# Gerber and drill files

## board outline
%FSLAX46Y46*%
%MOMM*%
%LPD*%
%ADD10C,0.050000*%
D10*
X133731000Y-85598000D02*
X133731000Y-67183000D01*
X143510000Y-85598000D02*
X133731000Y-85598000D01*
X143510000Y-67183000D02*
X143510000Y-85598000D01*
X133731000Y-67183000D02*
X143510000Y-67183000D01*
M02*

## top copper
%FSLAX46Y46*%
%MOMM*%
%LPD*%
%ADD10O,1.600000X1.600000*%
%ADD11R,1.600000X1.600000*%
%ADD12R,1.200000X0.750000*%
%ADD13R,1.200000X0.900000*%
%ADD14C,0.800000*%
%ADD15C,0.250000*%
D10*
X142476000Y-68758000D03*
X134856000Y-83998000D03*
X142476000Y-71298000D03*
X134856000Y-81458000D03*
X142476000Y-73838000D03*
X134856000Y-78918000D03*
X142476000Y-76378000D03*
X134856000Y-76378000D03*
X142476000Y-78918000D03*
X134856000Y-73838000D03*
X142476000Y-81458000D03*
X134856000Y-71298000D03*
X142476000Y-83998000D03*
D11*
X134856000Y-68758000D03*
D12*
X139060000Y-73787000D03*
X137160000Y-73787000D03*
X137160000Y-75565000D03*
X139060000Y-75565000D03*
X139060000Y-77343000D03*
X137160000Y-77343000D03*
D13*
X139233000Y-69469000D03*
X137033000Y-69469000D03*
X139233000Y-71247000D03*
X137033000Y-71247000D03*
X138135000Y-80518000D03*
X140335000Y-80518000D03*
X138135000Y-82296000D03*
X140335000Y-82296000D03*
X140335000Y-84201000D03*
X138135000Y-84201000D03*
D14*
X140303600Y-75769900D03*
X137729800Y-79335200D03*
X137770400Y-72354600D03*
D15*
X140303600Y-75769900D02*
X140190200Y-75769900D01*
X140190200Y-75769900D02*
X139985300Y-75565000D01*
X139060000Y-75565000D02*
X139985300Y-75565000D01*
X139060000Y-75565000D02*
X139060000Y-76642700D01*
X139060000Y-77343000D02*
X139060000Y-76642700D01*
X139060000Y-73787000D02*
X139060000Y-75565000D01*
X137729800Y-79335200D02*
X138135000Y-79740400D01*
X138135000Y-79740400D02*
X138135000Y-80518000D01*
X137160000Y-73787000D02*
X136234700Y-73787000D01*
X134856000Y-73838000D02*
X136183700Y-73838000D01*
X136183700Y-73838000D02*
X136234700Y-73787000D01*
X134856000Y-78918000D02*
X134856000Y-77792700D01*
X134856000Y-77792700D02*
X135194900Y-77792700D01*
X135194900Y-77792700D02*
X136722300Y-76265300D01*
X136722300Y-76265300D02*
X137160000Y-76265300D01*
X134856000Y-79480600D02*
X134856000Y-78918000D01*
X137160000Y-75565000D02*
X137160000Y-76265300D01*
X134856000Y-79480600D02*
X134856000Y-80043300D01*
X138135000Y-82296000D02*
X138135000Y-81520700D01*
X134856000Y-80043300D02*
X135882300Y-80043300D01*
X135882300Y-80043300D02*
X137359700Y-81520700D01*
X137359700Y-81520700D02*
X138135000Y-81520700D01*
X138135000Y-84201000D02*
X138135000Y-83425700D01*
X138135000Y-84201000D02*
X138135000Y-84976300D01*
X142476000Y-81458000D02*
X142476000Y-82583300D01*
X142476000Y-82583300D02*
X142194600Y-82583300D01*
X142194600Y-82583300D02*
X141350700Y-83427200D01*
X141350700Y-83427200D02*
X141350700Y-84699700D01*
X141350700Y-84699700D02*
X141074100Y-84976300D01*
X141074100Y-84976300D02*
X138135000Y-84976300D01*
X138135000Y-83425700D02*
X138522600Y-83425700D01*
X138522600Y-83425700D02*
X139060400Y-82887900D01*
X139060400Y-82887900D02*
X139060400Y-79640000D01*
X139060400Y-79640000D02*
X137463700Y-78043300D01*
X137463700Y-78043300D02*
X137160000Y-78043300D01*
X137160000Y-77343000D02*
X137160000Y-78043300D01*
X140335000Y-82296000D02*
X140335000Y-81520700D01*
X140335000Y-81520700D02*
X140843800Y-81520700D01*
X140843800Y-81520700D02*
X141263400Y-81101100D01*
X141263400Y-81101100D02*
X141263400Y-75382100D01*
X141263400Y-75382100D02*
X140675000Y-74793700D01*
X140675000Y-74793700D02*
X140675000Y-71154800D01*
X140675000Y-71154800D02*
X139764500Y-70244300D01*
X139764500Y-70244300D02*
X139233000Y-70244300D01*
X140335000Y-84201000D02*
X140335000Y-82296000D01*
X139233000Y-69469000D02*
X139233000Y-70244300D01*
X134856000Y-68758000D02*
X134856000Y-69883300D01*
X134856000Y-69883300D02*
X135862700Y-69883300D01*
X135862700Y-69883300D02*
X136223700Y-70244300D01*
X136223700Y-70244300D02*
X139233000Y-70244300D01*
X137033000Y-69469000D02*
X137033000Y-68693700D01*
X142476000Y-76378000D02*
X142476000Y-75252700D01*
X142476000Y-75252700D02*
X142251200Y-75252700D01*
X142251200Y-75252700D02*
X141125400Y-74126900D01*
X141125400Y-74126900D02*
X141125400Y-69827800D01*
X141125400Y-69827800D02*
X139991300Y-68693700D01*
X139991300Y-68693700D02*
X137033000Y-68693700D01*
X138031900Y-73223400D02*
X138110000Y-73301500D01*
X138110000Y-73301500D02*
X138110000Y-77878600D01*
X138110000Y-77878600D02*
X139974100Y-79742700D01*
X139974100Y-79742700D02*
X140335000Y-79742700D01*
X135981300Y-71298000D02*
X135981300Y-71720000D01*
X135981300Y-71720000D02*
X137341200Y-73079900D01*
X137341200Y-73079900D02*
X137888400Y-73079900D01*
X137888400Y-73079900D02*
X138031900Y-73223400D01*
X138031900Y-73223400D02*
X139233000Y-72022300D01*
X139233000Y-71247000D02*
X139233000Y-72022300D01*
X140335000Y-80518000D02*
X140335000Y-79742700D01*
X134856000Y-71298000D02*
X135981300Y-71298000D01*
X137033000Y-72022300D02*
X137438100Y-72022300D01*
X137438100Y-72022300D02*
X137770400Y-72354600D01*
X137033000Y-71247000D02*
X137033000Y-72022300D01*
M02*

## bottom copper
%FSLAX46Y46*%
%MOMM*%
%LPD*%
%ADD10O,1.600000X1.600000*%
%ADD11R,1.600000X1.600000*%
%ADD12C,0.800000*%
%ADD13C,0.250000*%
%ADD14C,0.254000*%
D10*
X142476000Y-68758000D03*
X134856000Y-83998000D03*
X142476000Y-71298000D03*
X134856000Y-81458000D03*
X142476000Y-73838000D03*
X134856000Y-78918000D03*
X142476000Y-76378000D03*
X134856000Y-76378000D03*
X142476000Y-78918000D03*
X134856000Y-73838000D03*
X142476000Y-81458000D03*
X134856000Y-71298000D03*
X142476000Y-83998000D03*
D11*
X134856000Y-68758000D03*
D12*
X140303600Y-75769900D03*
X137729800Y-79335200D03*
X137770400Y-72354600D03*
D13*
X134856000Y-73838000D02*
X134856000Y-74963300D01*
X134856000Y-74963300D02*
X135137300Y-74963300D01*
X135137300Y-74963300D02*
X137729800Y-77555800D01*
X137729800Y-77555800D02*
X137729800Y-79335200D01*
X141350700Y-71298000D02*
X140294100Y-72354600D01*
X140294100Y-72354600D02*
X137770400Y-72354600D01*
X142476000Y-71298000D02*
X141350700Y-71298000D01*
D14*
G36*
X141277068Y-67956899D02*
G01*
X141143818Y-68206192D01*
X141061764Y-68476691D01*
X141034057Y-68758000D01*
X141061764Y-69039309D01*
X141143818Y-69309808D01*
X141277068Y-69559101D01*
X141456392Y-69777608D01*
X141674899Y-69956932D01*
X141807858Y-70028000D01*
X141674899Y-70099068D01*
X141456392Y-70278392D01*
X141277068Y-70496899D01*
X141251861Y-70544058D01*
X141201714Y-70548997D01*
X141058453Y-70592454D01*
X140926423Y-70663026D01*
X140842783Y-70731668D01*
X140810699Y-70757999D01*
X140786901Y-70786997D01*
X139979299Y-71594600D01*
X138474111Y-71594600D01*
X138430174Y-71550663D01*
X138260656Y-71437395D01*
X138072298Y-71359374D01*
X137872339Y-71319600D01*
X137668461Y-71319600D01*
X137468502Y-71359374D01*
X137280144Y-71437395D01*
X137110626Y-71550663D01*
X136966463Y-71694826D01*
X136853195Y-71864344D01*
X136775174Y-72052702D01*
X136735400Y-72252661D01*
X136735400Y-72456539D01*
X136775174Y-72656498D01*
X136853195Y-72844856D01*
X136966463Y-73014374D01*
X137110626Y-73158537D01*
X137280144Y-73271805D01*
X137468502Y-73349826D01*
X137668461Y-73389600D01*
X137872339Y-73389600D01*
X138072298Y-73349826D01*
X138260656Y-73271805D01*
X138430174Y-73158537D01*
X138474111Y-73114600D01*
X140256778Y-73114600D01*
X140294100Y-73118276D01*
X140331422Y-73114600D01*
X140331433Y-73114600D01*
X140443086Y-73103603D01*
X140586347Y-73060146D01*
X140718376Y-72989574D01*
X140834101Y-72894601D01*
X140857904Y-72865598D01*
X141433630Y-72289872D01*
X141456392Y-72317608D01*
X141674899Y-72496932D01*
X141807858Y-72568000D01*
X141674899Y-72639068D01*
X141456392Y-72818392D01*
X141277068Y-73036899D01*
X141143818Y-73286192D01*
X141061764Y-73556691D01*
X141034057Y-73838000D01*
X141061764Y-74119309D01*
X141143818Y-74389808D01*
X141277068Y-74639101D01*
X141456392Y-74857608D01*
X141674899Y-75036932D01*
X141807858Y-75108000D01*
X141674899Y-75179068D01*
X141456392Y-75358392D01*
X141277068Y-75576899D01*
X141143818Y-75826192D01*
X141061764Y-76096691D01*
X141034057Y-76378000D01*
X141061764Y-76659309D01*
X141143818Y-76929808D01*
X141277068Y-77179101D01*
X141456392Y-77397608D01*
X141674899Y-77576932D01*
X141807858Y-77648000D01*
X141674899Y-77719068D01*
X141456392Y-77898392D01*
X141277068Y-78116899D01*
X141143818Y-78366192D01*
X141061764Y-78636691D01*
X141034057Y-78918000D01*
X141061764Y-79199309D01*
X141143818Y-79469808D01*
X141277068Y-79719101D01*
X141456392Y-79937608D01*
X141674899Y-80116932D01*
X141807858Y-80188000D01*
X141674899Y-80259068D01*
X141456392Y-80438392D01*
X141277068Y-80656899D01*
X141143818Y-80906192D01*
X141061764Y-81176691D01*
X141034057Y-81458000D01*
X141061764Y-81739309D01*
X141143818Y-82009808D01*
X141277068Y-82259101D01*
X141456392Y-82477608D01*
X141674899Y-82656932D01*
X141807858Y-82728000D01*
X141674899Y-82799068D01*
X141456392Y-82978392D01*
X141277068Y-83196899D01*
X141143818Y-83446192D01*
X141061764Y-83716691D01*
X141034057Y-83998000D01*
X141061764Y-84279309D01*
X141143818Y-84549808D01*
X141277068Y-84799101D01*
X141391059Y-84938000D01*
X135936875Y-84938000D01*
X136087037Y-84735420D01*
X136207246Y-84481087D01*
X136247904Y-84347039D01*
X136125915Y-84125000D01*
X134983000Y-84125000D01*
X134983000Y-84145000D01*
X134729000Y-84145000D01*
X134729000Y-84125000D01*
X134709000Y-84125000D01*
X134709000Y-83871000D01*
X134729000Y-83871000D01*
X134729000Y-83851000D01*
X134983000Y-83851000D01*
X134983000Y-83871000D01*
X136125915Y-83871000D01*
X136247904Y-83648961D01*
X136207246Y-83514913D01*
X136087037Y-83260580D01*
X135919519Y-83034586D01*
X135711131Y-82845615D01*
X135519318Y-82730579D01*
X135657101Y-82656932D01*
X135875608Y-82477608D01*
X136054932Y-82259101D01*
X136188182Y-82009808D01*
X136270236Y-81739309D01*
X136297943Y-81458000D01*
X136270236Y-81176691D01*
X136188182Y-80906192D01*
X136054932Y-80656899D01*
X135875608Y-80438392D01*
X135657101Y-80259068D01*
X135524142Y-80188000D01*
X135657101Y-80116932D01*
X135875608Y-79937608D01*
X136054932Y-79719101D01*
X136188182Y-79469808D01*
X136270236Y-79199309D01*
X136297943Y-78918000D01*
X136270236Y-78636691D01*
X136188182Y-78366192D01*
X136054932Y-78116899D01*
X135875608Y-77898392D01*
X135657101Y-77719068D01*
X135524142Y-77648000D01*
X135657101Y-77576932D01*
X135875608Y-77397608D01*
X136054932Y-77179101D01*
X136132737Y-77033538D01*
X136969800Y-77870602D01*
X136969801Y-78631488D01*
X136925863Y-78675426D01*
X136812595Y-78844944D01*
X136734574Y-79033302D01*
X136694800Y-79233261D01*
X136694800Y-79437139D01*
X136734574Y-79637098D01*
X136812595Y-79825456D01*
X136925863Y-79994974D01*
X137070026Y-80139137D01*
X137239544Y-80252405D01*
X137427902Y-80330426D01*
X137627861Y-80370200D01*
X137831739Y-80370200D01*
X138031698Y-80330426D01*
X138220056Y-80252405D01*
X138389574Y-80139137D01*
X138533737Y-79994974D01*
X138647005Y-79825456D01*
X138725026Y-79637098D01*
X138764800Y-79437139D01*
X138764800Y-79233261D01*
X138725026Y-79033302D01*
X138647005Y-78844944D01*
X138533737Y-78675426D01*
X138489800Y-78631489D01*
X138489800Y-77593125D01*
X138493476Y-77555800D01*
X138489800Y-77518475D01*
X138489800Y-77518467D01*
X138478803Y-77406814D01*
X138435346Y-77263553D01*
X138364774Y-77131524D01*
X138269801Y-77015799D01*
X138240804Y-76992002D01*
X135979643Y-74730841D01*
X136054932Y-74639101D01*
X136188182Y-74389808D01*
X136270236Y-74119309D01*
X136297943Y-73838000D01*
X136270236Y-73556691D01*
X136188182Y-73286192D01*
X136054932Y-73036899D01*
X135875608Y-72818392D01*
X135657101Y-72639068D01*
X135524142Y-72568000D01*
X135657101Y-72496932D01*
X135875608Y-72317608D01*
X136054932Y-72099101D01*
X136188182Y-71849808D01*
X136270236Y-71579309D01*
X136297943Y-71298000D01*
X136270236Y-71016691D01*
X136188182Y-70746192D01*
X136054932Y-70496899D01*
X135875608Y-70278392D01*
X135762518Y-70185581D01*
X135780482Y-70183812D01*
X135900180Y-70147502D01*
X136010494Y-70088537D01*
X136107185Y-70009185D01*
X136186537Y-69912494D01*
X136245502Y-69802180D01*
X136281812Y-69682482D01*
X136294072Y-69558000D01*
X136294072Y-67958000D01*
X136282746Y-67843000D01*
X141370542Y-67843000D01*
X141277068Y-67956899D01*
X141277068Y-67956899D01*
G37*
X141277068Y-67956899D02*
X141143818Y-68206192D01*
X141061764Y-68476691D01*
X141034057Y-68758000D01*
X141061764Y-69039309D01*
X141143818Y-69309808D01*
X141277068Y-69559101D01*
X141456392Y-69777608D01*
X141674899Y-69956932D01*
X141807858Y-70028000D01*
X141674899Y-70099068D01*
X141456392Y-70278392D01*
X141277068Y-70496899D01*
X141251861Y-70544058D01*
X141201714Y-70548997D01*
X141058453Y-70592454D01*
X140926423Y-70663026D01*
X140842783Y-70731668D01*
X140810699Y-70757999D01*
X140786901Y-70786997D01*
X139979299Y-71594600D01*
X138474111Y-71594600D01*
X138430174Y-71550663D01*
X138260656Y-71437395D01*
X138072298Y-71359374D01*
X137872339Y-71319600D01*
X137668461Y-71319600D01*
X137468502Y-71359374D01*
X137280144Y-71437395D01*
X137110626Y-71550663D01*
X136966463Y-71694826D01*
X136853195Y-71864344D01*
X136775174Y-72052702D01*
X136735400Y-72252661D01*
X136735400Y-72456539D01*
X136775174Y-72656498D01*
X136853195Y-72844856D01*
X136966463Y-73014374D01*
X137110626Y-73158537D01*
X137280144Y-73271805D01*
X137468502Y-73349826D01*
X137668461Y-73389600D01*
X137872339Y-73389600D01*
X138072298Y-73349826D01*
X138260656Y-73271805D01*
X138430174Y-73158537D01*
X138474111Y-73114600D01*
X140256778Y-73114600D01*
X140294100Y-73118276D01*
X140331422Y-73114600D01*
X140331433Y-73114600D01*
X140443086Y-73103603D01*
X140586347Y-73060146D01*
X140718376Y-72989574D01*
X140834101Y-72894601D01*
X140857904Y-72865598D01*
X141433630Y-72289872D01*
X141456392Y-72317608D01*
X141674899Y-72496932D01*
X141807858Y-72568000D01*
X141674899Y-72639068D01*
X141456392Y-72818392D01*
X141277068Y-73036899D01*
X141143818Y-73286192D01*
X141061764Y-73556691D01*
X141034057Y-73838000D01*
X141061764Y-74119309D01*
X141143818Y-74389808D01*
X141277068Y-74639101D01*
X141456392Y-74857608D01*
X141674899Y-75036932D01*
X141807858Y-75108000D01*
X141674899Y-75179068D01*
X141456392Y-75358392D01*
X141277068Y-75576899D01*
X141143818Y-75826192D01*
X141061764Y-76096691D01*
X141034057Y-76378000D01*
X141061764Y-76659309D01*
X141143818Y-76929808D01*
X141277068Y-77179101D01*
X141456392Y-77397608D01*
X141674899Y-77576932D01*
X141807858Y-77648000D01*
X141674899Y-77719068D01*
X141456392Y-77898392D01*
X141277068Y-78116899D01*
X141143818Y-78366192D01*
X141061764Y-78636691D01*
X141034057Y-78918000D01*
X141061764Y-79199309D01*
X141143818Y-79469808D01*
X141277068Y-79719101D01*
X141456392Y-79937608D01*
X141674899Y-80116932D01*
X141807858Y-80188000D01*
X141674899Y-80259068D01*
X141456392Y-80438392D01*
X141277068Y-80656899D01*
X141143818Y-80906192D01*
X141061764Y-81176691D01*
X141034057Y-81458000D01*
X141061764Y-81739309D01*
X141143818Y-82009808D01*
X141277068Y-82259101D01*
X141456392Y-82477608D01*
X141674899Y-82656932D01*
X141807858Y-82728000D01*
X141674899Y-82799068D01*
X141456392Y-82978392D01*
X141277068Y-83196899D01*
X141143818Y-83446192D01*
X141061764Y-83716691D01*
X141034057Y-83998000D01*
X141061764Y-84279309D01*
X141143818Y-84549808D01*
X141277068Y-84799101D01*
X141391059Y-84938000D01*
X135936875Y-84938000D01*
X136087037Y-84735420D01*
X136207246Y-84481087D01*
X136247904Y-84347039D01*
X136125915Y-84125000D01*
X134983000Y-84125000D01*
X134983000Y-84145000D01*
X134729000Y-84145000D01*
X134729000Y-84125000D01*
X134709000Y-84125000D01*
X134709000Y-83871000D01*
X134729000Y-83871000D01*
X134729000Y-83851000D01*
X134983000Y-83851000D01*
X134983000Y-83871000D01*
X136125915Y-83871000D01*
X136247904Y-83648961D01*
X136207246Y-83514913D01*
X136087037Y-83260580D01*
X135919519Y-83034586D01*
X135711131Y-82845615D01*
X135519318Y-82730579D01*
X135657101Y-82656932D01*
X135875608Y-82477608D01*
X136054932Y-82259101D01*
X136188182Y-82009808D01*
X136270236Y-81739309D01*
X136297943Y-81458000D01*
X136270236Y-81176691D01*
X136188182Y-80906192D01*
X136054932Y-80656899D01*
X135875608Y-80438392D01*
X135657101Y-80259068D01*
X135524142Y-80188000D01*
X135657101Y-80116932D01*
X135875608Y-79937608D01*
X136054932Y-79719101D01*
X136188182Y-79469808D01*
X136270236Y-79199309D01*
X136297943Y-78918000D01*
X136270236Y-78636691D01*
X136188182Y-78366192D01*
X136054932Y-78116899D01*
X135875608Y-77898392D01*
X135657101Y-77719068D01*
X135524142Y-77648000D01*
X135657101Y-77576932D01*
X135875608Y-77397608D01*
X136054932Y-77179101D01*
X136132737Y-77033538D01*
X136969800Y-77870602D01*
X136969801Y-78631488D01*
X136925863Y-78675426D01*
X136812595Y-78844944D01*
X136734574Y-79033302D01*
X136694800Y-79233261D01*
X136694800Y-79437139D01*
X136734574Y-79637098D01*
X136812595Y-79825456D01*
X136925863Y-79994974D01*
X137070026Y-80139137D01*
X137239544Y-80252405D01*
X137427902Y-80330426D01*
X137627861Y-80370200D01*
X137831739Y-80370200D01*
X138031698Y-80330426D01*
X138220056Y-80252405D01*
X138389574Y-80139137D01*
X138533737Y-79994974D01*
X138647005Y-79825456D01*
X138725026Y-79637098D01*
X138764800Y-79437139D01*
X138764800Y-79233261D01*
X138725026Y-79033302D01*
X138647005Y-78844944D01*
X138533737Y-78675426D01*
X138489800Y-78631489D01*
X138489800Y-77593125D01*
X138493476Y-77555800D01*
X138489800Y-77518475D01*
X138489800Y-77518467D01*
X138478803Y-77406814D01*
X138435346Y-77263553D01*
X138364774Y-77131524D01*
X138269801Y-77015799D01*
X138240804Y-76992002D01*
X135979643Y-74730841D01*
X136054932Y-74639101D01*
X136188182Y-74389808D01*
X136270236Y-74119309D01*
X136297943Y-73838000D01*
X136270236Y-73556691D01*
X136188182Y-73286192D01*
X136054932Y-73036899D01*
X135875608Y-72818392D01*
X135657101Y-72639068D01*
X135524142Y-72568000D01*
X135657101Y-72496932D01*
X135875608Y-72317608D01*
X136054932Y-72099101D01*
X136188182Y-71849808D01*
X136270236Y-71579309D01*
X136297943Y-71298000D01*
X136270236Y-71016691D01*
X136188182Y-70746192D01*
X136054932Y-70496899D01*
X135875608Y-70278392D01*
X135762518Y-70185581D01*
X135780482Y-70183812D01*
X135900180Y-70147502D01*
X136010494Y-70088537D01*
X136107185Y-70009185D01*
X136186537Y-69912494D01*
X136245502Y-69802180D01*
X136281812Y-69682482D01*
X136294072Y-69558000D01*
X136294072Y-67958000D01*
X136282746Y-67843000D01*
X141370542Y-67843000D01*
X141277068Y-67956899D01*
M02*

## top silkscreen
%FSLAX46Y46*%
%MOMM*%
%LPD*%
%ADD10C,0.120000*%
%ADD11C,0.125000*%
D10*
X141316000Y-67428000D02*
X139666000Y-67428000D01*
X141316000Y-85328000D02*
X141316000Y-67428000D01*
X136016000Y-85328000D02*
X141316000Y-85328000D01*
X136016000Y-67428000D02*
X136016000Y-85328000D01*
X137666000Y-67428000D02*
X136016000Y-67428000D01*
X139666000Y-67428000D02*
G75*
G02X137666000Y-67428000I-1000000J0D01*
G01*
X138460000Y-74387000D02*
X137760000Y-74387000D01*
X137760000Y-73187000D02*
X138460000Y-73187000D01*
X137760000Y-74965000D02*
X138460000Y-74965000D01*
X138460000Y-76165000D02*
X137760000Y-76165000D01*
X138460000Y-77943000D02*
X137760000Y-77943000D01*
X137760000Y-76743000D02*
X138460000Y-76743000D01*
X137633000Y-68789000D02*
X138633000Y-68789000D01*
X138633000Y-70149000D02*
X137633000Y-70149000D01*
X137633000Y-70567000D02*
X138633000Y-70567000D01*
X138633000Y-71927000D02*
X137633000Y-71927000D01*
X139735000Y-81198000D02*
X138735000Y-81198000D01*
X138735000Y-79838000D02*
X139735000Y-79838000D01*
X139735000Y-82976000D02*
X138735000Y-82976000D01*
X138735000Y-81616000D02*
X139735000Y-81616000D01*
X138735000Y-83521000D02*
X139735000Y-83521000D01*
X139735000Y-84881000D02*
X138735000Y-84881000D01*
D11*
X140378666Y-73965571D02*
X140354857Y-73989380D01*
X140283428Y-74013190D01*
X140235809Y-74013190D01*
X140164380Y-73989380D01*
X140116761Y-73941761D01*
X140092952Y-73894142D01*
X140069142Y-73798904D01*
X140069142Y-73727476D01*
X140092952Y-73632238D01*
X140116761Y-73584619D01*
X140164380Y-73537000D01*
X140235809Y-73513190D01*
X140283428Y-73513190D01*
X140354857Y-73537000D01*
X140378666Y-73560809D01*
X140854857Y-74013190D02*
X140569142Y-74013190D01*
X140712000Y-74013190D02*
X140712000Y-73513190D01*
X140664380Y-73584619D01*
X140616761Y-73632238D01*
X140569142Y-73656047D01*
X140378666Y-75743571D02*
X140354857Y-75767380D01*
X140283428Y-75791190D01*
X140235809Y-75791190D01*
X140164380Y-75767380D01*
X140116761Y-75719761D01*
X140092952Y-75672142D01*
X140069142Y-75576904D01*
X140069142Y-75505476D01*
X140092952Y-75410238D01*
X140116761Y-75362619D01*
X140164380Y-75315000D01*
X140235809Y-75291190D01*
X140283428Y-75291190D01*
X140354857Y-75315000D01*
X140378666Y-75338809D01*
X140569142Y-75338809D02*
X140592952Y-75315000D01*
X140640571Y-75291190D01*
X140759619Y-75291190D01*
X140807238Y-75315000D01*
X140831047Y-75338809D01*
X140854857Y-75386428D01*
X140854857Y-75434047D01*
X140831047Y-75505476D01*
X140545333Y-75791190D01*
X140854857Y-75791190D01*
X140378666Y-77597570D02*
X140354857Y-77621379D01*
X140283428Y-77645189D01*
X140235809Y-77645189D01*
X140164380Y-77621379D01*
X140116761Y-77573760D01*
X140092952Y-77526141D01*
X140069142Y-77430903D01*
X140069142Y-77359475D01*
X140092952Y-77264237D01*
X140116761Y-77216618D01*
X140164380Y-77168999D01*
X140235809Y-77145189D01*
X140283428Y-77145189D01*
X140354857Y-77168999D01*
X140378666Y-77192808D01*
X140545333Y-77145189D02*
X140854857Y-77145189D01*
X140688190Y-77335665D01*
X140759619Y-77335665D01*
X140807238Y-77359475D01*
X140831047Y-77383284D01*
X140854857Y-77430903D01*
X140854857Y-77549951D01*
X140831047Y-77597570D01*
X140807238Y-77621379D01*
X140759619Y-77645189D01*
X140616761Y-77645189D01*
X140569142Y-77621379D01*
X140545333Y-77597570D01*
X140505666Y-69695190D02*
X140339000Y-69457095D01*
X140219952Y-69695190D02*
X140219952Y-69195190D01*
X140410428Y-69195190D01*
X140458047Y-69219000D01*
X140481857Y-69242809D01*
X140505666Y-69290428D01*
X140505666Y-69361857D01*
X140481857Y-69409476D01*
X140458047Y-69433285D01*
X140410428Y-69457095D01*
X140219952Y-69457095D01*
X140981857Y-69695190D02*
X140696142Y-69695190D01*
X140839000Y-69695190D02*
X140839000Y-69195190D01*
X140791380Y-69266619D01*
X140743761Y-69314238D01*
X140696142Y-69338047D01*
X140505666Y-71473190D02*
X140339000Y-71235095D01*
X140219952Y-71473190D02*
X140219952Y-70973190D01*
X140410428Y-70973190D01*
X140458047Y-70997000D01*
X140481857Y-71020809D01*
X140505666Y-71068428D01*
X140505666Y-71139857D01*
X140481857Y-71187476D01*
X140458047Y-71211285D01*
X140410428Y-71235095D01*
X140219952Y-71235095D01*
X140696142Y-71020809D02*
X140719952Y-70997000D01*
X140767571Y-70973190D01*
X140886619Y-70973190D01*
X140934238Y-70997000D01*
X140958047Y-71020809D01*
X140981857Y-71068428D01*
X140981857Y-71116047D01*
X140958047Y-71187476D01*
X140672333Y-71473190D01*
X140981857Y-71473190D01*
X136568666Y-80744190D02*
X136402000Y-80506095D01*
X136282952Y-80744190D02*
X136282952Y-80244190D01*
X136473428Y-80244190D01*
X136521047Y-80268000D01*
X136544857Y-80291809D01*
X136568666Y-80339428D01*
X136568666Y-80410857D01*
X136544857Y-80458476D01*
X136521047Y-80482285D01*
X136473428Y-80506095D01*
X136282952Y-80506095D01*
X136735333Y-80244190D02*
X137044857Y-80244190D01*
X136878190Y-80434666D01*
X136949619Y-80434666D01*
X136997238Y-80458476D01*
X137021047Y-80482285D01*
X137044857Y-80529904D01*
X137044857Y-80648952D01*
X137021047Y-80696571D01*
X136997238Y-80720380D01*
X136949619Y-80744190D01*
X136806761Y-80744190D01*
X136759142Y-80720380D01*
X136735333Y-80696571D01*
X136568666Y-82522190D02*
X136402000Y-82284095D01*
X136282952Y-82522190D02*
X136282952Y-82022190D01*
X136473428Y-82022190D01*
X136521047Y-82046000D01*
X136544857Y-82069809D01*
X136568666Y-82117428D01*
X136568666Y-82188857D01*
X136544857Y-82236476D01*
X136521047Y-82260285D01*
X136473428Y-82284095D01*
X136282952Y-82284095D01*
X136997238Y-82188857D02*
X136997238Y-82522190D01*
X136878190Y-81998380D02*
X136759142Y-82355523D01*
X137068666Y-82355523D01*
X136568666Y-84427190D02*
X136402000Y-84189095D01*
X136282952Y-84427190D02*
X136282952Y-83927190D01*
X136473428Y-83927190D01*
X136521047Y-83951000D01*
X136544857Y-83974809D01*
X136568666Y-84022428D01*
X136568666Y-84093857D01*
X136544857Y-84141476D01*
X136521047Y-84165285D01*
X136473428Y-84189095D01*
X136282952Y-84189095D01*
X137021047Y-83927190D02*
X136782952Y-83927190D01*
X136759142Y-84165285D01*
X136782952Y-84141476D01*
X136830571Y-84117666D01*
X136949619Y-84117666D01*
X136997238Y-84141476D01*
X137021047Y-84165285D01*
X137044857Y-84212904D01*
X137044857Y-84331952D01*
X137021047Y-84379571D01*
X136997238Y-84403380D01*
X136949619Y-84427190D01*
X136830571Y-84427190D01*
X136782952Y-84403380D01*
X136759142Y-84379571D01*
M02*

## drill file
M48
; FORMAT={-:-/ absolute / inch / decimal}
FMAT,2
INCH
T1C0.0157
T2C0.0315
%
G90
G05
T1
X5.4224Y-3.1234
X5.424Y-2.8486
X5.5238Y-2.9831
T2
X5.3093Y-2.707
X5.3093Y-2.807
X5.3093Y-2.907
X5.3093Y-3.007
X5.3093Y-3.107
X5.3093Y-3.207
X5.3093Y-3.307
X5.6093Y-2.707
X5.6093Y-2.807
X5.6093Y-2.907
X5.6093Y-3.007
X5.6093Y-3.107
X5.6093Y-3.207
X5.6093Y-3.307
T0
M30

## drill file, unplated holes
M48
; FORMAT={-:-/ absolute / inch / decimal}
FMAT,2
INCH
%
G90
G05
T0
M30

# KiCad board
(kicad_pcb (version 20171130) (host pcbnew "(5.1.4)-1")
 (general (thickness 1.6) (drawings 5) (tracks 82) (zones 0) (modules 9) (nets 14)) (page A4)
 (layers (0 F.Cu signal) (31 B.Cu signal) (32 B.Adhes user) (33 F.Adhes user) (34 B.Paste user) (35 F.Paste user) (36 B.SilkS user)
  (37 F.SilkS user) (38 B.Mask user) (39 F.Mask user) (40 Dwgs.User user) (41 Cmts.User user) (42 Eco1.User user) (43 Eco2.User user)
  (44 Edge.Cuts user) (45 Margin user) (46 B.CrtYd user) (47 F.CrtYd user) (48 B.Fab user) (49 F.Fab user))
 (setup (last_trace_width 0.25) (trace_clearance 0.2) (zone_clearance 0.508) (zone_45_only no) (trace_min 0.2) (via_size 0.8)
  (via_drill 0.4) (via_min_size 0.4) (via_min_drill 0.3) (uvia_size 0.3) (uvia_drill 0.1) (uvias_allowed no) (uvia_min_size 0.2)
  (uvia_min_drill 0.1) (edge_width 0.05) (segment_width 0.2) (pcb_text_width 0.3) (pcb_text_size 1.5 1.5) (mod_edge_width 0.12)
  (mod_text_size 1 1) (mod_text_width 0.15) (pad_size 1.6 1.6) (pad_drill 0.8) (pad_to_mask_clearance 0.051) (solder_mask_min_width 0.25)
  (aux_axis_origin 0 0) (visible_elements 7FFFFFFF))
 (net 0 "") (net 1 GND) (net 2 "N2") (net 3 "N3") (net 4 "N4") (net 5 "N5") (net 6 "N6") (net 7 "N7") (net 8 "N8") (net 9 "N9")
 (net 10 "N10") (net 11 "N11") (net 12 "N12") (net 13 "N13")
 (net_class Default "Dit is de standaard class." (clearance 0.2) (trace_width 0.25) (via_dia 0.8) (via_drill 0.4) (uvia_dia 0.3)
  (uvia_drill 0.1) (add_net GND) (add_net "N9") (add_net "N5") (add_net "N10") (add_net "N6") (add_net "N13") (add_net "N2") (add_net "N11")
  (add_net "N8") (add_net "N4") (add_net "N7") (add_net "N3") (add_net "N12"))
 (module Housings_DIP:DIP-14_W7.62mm (layer F.Cu) (at 134.856 68.758)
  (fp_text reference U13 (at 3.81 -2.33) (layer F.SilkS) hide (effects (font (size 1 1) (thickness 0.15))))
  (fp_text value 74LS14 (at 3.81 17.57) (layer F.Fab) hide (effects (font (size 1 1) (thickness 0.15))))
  (fp_line (start 6.46 -1.33) (end 4.81 -1.33) (layer F.SilkS) (width 0.12))
  (fp_line (start 6.46 16.57) (end 6.46 -1.33) (layer F.SilkS) (width 0.12))
  (fp_line (start 1.16 16.57) (end 6.46 16.57) (layer F.SilkS) (width 0.12))
  (fp_line (start 1.16 -1.33) (end 1.16 16.57) (layer F.SilkS) (width 0.12))
  (fp_line (start 2.81 -1.33) (end 1.16 -1.33) (layer F.SilkS) (width 0.12))
  (fp_arc (start 3.81 -1.33) (end 2.81 -1.33) (angle -180) (layer F.SilkS) (width 0.12))
  (pad 14 thru_hole oval (at 7.62 0) (size 1.6 1.6) (drill 0.8) (layers *.Cu *.Mask))
  (pad 7 thru_hole oval (at 0 15.24) (size 1.6 1.6) (drill 0.8) (layers *.Cu *.Mask) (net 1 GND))
  (pad 13 thru_hole oval (at 7.62 2.54) (size 1.6 1.6) (drill 0.8) (layers *.Cu *.Mask) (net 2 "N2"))
  (pad 6 thru_hole oval (at 0 12.7) (size 1.6 1.6) (drill 0.8) (layers *.Cu *.Mask) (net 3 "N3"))
  (pad 12 thru_hole oval (at 7.62 5.08) (size 1.6 1.6) (drill 0.8) (layers *.Cu *.Mask) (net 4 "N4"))
  (pad 5 thru_hole oval (at 0 10.16) (size 1.6 1.6) (drill 0.8) (layers *.Cu *.Mask) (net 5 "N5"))
  (pad 11 thru_hole oval (at 7.62 7.62) (size 1.6 1.6) (drill 0.8) (layers *.Cu *.Mask) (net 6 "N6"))
  (pad 4 thru_hole oval (at 0 7.62) (size 1.6 1.6) (drill 0.8) (layers *.Cu *.Mask) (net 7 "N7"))
  (pad 10 thru_hole oval (at 7.62 10.16) (size 1.6 1.6) (drill 0.8) (layers *.Cu *.Mask) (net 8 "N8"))
  (pad 3 thru_hole oval (at 0 5.08) (size 1.6 1.6) (drill 0.8) (layers *.Cu *.Mask) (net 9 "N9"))
  (pad 9 thru_hole oval (at 7.62 12.7) (size 1.6 1.6) (drill 0.8) (layers *.Cu *.Mask) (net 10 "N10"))
  (pad 2 thru_hole oval (at 0 2.54) (size 1.6 1.6) (drill 0.8) (layers *.Cu *.Mask) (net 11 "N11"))
  (pad 8 thru_hole oval (at 7.62 15.24) (size 1.6 1.6) (drill 0.8) (layers *.Cu *.Mask) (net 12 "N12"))
  (pad 1 thru_hole rect (at 0 0) (size 1.6 1.6) (drill 0.8) (layers *.Cu *.Mask) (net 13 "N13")))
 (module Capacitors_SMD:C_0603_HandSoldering (layer F.Cu) (at 138.11 73.787)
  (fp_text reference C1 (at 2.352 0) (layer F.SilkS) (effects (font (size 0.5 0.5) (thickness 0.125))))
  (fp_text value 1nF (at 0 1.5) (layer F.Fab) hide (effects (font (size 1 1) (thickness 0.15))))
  (fp_line (start 0.35 0.6) (end -0.35 0.6) (layer F.SilkS) (width 0.12))
  (fp_line (start -0.35 -0.6) (end 0.35 -0.6) (layer F.SilkS) (width 0.12))
  (pad 2 smd rect (at 0.95 0) (size 1.2 0.75) (layers F.Cu F.Paste F.Mask) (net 1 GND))
  (pad 1 smd rect (at -0.95 0) (size 1.2 0.75) (layers F.Cu F.Paste F.Mask) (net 9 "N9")))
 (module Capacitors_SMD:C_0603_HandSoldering (layer F.Cu) (at 138.11 75.565)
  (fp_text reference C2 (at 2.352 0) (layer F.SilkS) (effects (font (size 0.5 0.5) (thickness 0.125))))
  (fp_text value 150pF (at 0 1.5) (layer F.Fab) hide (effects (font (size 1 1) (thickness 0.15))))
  (fp_line (start -0.35 -0.6) (end 0.35 -0.6) (layer F.SilkS) (width 0.12))
  (fp_line (start 0.35 0.6) (end -0.35 0.6) (layer F.SilkS) (width 0.12))
  (pad 1 smd rect (at -0.95 0) (size 1.2 0.75) (layers F.Cu F.Paste F.Mask) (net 5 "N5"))
  (pad 2 smd rect (at 0.95 0) (size 1.2 0.75) (layers F.Cu F.Paste F.Mask) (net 1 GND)))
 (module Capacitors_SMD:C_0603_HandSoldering (layer F.Cu) (at 138.11 77.343)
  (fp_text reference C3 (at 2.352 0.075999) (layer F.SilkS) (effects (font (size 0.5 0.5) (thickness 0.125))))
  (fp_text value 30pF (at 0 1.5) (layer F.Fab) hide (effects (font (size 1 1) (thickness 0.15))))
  (fp_line (start 0.35 0.6) (end -0.35 0.6) (layer F.SilkS) (width 0.12))
  (fp_line (start -0.35 -0.6) (end 0.35 -0.6) (layer F.SilkS) (width 0.12))
  (pad 2 smd rect (at 0.95 0) (size 1.2 0.75) (layers F.Cu F.Paste F.Mask) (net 1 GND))
  (pad 1 smd rect (at -0.95 0) (size 1.2 0.75) (layers F.Cu F.Paste F.Mask) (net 10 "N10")))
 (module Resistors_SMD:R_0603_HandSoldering (layer F.Cu) (at 138.133 69.469)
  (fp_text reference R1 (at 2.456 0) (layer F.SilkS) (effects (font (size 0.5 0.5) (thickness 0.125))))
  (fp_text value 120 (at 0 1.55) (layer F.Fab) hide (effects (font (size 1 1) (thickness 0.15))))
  (fp_line (start -0.5 -0.68) (end 0.5 -0.68) (layer F.SilkS) (width 0.12))
  (fp_line (start 0.5 0.68) (end -0.5 0.68) (layer F.SilkS) (width 0.12))
  (pad 2 smd rect (at 1.1 0) (size 1.2 0.9) (layers F.Cu F.Paste F.Mask) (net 13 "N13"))
  (pad 1 smd rect (at -1.1 0) (size 1.2 0.9) (layers F.Cu F.Paste F.Mask) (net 6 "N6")))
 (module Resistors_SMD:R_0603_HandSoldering (layer F.Cu) (at 138.133 71.247)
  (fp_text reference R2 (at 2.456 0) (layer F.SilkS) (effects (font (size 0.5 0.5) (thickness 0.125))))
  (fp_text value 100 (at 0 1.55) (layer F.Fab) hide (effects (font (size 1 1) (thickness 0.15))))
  (fp_line (start -0.5 -0.68) (end 0.5 -0.68) (layer F.SilkS) (width 0.12))
  (fp_line (start 0.5 0.68) (end -0.5 0.68) (layer F.SilkS) (width 0.12))
  (pad 2 smd rect (at 1.1 0) (size 1.2 0.9) (layers F.Cu F.Paste F.Mask) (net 11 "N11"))
  (pad 1 smd rect (at -1.1 0) (size 1.2 0.9) (layers F.Cu F.Paste F.Mask) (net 2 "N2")))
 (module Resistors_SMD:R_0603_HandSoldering (layer F.Cu) (at 139.235 80.518)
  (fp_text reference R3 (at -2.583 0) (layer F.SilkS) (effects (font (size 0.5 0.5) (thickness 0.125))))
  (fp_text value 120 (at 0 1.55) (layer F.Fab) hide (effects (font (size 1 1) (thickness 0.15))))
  (fp_line (start 0.5 0.68) (end -0.5 0.68) (layer F.SilkS) (width 0.12))
  (fp_line (start -0.5 -0.68) (end 0.5 -0.68) (layer F.SilkS) (width 0.12))
  (pad 1 smd rect (at -1.1 0) (size 1.2 0.9) (layers F.Cu F.Paste F.Mask) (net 9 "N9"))
  (pad 2 smd rect (at 1.1 0) (size 1.2 0.9) (layers F.Cu F.Paste F.Mask) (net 11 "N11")))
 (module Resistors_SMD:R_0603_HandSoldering (layer F.Cu) (at 139.235 82.296)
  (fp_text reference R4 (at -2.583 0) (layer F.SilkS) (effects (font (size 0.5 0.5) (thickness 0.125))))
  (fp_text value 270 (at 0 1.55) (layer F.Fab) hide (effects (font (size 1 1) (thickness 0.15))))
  (fp_line (start 0.5 0.68) (end -0.5 0.68) (layer F.SilkS) (width 0.12))
  (fp_line (start -0.5 -0.68) (end 0.5 -0.68) (layer F.SilkS) (width 0.12))
  (pad 1 smd rect (at -1.1 0) (size 1.2 0.9) (layers F.Cu F.Paste F.Mask) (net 5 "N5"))
  (pad 2 smd rect (at 1.1 0) (size 1.2 0.9) (layers F.Cu F.Paste F.Mask) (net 13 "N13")))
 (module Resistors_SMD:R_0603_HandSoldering (layer F.Cu) (at 139.235 84.201)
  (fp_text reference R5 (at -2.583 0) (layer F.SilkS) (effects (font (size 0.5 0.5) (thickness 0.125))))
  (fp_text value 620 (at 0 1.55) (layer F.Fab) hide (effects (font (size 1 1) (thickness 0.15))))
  (fp_line (start -0.5 -0.68) (end 0.5 -0.68) (layer F.SilkS) (width 0.12))
  (fp_line (start 0.5 0.68) (end -0.5 0.68) (layer F.SilkS) (width 0.12))
  (pad 2 smd rect (at 1.1 0) (size 1.2 0.9) (layers F.Cu F.Paste F.Mask) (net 13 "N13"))
  (pad 1 smd rect (at -1.1 0) (size 1.2 0.9) (layers F.Cu F.Paste F.Mask) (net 10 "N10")))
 (gr_line (start 133.731 85.598) (end 133.731 67.183) (layer Edge.Cuts) (width 0.05))
 (gr_line (start 143.51 85.598) (end 133.731 85.598) (layer Edge.Cuts) (width 0.05))
 (gr_line (start 143.51 67.183) (end 143.51 85.598) (layer Edge.Cuts) (width 0.05))
 (gr_line (start 133.731 67.183) (end 143.51 67.183) (layer Edge.Cuts) (width 0.05))
 (segment (start 140.3036 75.7699) (end 140.1902 75.7699) (width 0.25) (layer F.Cu) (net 1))
 (segment (start 140.1902 75.7699) (end 139.9853 75.565) (width 0.25) (layer F.Cu) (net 1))
 (segment (start 139.06 75.565) (end 139.9853 75.565) (width 0.25) (layer F.Cu) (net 1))
 (segment (start 139.06 75.565) (end 139.06 76.6427) (width 0.25) (layer F.Cu) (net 1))
 (segment (start 139.06 77.343) (end 139.06 76.6427) (width 0.25) (layer F.Cu) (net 1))
 (segment (start 139.06 73.787) (end 139.06 75.565) (width 0.25) (layer F.Cu) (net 1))
 (via (at 140.3036 75.7699) (size 0.8) (layers F.Cu B.Cu) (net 1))
 (segment (start 134.856 73.838) (end 134.856 74.9633) (width 0.25) (layer B.Cu) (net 9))
 (segment (start 137.7298 79.3352) (end 138.135 79.7404) (width 0.25) (layer F.Cu) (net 9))
 (segment (start 138.135 79.7404) (end 138.135 80.518) (width 0.25) (layer F.Cu) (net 9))
 (segment (start 134.856 74.9633) (end 135.1373 74.9633) (width 0.25) (layer B.Cu) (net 9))
 (segment (start 135.1373 74.9633) (end 137.7298 77.5558) (width 0.25) (layer B.Cu) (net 9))
 (segment (start 137.7298 77.5558) (end 137.7298 79.3352) (width 0.25) (layer B.Cu) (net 9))
 (segment (start 137.16 73.787) (end 136.2347 73.787) (width 0.25) (layer F.Cu) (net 9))
 (segment (start 134.856 73.838) (end 136.1837 73.838) (width 0.25) (layer F.Cu) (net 9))
 (segment (start 136.1837 73.838) (end 136.2347 73.787) (width 0.25) (layer F.Cu) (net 9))
 (via (at 137.7298 79.3352) (size 0.8) (layers F.Cu B.Cu) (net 9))
 (segment (start 134.856 78.918) (end 134.856 77.7927) (width 0.25) (layer F.Cu) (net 5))
 (segment (start 134.856 77.7927) (end 135.1949 77.7927) (width 0.25) (layer F.Cu) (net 5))
 (segment (start 135.1949 77.7927) (end 136.7223 76.2653) (width 0.25) (layer F.Cu) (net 5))
 (segment (start 136.7223 76.2653) (end 137.16 76.2653) (width 0.25) (layer F.Cu) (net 5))
 (segment (start 134.856 79.4806) (end 134.856 78.918) (width 0.25) (layer F.Cu) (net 5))
 (segment (start 137.16 75.565) (end 137.16 76.2653) (width 0.25) (layer F.Cu) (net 5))
 (segment (start 134.856 79.4806) (end 134.856 80.0433) (width 0.25) (layer F.Cu) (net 5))
 (segment (start 138.135 82.296) (end 138.135 81.5207) (width 0.25) (layer F.Cu) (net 5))
 (segment (start 134.856 80.0433) (end 135.8823 80.0433) (width 0.25) (layer F.Cu) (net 5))
 (segment (start 135.8823 80.0433) (end 137.3597 81.5207) (width 0.25) (layer F.Cu) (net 5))
 (segment (start 137.3597 81.5207) (end 138.135 81.5207) (width 0.25) (layer F.Cu) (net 5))
 (segment (start 138.135 84.201) (end 138.135 83.4257) (width 0.25) (layer F.Cu) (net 10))
 (segment (start 138.135 84.201) (end 138.135 84.9763) (width 0.25) (layer F.Cu) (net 10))
 (segment (start 142.476 81.458) (end 142.476 82.5833) (width 0.25) (layer F.Cu) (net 10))
 (segment (start 142.476 82.5833) (end 142.1946 82.5833) (width 0.25) (layer F.Cu) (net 10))
 (segment (start 142.1946 82.5833) (end 141.3507 83.4272) (width 0.25) (layer F.Cu) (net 10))
 (segment (start 141.3507 83.4272) (end 141.3507 84.6997) (width 0.25) (layer F.Cu) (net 10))
 (segment (start 141.3507 84.6997) (end 141.0741 84.9763) (width 0.25) (layer F.Cu) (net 10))
 (segment (start 141.0741 84.9763) (end 138.135 84.9763) (width 0.25) (layer F.Cu) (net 10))
 (segment (start 138.135 83.4257) (end 138.5226 83.4257) (width 0.25) (layer F.Cu) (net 10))
 (segment (start 138.5226 83.4257) (end 139.0604 82.8879) (width 0.25) (layer F.Cu) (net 10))
 (segment (start 139.0604 82.8879) (end 139.0604 79.64) (width 0.25) (layer F.Cu) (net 10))
 (segment (start 139.0604 79.64) (end 137.4637 78.0433) (width 0.25) (layer F.Cu) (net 10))
 (segment (start 137.4637 78.0433) (end 137.16 78.0433) (width 0.25) (layer F.Cu) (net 10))
 (segment (start 137.16 77.343) (end 137.16 78.0433) (width 0.25) (layer F.Cu) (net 10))
 (segment (start 140.335 82.296) (end 140.335 81.5207) (width 0.25) (layer F.Cu) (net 13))
 (segment (start 140.335 81.5207) (end 140.8438 81.5207) (width 0.25) (layer F.Cu) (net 13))
 (segment (start 140.8438 81.5207) (end 141.2634 81.1011) (width 0.25) (layer F.Cu) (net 13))
 (segment (start 141.2634 81.1011) (end 141.2634 75.3821) (width 0.25) (layer F.Cu) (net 13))
 (segment (start 141.2634 75.3821) (end 140.675 74.7937) (width 0.25) (layer F.Cu) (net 13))
 (segment (start 140.675 74.7937) (end 140.675 71.1548) (width 0.25) (layer F.Cu) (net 13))
 (segment (start 140.675 71.1548) (end 139.7645 70.2443) (width 0.25) (layer F.Cu) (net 13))
 (segment (start 139.7645 70.2443) (end 139.233 70.2443) (width 0.25) (layer F.Cu) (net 13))
 (segment (start 140.335 84.201) (end 140.335 82.296) (width 0.25) (layer F.Cu) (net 13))
 (segment (start 139.233 69.469) (end 139.233 70.2443) (width 0.25) (layer F.Cu) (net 13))
 (segment (start 134.856 68.758) (end 134.856 69.8833) (width 0.25) (layer F.Cu) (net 13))
 (segment (start 134.856 69.8833) (end 135.8627 69.8833) (width 0.25) (layer F.Cu) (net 13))
 (segment (start 135.8627 69.8833) (end 136.2237 70.2443) (width 0.25) (layer F.Cu) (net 13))
 (segment (start 136.2237 70.2443) (end 139.233 70.2443) (width 0.25) (layer F.Cu) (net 13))
 (segment (start 137.033 69.469) (end 137.033 68.6937) (width 0.25) (layer F.Cu) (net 6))
 (segment (start 142.476 76.378) (end 142.476 75.2527) (width 0.25) (layer F.Cu) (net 6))
 (segment (start 142.476 75.2527) (end 142.2512 75.2527) (width 0.25) (layer F.Cu) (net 6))
 (segment (start 142.2512 75.2527) (end 141.1254 74.1269) (width 0.25) (layer F.Cu) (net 6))
 (segment (start 141.1254 74.1269) (end 141.1254 69.8278) (width 0.25) (layer F.Cu) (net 6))
 (segment (start 141.1254 69.8278) (end 139.9913 68.6937) (width 0.25) (layer F.Cu) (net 6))
 (segment (start 139.9913 68.6937) (end 137.033 68.6937) (width 0.25) (layer F.Cu) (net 6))
 (segment (start 138.0319 73.2234) (end 138.11 73.3015) (width 0.25) (layer F.Cu) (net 11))
 (segment (start 138.11 73.3015) (end 138.11 77.8786) (width 0.25) (layer F.Cu) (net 11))
 (segment (start 138.11 77.8786) (end 139.9741 79.7427) (width 0.25) (layer F.Cu) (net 11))
 (segment (start 139.9741 79.7427) (end 140.335 79.7427) (width 0.25) (layer F.Cu) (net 11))
 (segment (start 135.9813 71.298) (end 135.9813 71.72) (width 0.25) (layer F.Cu) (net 11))
 (segment (start 135.9813 71.72) (end 137.3412 73.0799) (width 0.25) (layer F.Cu) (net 11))
 (segment (start 137.3412 73.0799) (end 137.8884 73.0799) (width 0.25) (layer F.Cu) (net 11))
 (segment (start 137.8884 73.0799) (end 138.0319 73.2234) (width 0.25) (layer F.Cu) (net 11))
 (segment (start 138.0319 73.2234) (end 139.233 72.0223) (width 0.25) (layer F.Cu) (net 11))
 (segment (start 139.233 71.247) (end 139.233 72.0223) (width 0.25) (layer F.Cu) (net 11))
 (segment (start 140.335 80.518) (end 140.335 79.7427) (width 0.25) (layer F.Cu) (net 11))
 (segment (start 134.856 71.298) (end 135.9813 71.298) (width 0.25) (layer F.Cu) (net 11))
 (segment (start 137.033 72.0223) (end 137.4381 72.0223) (width 0.25) (layer F.Cu) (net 2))
 (segment (start 137.4381 72.0223) (end 137.7704 72.3546) (width 0.25) (layer F.Cu) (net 2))
 (segment (start 141.3507 71.298) (end 140.2941 72.3546) (width 0.25) (layer B.Cu) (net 2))
 (segment (start 140.2941 72.3546) (end 137.7704 72.3546) (width 0.25) (layer B.Cu) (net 2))
 (segment (start 137.033 71.247) (end 137.033 72.0223) (width 0.25) (layer F.Cu) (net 2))
 (segment (start 142.476 71.298) (end 141.3507 71.298) (width 0.25) (layer B.Cu) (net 2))
 (via (at 137.7704 72.3546) (size 0.8) (layers F.Cu B.Cu) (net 2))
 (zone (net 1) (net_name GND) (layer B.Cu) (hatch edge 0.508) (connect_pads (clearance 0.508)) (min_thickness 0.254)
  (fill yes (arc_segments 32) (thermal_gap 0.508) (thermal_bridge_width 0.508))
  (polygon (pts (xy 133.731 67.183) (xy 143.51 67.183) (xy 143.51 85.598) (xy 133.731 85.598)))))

